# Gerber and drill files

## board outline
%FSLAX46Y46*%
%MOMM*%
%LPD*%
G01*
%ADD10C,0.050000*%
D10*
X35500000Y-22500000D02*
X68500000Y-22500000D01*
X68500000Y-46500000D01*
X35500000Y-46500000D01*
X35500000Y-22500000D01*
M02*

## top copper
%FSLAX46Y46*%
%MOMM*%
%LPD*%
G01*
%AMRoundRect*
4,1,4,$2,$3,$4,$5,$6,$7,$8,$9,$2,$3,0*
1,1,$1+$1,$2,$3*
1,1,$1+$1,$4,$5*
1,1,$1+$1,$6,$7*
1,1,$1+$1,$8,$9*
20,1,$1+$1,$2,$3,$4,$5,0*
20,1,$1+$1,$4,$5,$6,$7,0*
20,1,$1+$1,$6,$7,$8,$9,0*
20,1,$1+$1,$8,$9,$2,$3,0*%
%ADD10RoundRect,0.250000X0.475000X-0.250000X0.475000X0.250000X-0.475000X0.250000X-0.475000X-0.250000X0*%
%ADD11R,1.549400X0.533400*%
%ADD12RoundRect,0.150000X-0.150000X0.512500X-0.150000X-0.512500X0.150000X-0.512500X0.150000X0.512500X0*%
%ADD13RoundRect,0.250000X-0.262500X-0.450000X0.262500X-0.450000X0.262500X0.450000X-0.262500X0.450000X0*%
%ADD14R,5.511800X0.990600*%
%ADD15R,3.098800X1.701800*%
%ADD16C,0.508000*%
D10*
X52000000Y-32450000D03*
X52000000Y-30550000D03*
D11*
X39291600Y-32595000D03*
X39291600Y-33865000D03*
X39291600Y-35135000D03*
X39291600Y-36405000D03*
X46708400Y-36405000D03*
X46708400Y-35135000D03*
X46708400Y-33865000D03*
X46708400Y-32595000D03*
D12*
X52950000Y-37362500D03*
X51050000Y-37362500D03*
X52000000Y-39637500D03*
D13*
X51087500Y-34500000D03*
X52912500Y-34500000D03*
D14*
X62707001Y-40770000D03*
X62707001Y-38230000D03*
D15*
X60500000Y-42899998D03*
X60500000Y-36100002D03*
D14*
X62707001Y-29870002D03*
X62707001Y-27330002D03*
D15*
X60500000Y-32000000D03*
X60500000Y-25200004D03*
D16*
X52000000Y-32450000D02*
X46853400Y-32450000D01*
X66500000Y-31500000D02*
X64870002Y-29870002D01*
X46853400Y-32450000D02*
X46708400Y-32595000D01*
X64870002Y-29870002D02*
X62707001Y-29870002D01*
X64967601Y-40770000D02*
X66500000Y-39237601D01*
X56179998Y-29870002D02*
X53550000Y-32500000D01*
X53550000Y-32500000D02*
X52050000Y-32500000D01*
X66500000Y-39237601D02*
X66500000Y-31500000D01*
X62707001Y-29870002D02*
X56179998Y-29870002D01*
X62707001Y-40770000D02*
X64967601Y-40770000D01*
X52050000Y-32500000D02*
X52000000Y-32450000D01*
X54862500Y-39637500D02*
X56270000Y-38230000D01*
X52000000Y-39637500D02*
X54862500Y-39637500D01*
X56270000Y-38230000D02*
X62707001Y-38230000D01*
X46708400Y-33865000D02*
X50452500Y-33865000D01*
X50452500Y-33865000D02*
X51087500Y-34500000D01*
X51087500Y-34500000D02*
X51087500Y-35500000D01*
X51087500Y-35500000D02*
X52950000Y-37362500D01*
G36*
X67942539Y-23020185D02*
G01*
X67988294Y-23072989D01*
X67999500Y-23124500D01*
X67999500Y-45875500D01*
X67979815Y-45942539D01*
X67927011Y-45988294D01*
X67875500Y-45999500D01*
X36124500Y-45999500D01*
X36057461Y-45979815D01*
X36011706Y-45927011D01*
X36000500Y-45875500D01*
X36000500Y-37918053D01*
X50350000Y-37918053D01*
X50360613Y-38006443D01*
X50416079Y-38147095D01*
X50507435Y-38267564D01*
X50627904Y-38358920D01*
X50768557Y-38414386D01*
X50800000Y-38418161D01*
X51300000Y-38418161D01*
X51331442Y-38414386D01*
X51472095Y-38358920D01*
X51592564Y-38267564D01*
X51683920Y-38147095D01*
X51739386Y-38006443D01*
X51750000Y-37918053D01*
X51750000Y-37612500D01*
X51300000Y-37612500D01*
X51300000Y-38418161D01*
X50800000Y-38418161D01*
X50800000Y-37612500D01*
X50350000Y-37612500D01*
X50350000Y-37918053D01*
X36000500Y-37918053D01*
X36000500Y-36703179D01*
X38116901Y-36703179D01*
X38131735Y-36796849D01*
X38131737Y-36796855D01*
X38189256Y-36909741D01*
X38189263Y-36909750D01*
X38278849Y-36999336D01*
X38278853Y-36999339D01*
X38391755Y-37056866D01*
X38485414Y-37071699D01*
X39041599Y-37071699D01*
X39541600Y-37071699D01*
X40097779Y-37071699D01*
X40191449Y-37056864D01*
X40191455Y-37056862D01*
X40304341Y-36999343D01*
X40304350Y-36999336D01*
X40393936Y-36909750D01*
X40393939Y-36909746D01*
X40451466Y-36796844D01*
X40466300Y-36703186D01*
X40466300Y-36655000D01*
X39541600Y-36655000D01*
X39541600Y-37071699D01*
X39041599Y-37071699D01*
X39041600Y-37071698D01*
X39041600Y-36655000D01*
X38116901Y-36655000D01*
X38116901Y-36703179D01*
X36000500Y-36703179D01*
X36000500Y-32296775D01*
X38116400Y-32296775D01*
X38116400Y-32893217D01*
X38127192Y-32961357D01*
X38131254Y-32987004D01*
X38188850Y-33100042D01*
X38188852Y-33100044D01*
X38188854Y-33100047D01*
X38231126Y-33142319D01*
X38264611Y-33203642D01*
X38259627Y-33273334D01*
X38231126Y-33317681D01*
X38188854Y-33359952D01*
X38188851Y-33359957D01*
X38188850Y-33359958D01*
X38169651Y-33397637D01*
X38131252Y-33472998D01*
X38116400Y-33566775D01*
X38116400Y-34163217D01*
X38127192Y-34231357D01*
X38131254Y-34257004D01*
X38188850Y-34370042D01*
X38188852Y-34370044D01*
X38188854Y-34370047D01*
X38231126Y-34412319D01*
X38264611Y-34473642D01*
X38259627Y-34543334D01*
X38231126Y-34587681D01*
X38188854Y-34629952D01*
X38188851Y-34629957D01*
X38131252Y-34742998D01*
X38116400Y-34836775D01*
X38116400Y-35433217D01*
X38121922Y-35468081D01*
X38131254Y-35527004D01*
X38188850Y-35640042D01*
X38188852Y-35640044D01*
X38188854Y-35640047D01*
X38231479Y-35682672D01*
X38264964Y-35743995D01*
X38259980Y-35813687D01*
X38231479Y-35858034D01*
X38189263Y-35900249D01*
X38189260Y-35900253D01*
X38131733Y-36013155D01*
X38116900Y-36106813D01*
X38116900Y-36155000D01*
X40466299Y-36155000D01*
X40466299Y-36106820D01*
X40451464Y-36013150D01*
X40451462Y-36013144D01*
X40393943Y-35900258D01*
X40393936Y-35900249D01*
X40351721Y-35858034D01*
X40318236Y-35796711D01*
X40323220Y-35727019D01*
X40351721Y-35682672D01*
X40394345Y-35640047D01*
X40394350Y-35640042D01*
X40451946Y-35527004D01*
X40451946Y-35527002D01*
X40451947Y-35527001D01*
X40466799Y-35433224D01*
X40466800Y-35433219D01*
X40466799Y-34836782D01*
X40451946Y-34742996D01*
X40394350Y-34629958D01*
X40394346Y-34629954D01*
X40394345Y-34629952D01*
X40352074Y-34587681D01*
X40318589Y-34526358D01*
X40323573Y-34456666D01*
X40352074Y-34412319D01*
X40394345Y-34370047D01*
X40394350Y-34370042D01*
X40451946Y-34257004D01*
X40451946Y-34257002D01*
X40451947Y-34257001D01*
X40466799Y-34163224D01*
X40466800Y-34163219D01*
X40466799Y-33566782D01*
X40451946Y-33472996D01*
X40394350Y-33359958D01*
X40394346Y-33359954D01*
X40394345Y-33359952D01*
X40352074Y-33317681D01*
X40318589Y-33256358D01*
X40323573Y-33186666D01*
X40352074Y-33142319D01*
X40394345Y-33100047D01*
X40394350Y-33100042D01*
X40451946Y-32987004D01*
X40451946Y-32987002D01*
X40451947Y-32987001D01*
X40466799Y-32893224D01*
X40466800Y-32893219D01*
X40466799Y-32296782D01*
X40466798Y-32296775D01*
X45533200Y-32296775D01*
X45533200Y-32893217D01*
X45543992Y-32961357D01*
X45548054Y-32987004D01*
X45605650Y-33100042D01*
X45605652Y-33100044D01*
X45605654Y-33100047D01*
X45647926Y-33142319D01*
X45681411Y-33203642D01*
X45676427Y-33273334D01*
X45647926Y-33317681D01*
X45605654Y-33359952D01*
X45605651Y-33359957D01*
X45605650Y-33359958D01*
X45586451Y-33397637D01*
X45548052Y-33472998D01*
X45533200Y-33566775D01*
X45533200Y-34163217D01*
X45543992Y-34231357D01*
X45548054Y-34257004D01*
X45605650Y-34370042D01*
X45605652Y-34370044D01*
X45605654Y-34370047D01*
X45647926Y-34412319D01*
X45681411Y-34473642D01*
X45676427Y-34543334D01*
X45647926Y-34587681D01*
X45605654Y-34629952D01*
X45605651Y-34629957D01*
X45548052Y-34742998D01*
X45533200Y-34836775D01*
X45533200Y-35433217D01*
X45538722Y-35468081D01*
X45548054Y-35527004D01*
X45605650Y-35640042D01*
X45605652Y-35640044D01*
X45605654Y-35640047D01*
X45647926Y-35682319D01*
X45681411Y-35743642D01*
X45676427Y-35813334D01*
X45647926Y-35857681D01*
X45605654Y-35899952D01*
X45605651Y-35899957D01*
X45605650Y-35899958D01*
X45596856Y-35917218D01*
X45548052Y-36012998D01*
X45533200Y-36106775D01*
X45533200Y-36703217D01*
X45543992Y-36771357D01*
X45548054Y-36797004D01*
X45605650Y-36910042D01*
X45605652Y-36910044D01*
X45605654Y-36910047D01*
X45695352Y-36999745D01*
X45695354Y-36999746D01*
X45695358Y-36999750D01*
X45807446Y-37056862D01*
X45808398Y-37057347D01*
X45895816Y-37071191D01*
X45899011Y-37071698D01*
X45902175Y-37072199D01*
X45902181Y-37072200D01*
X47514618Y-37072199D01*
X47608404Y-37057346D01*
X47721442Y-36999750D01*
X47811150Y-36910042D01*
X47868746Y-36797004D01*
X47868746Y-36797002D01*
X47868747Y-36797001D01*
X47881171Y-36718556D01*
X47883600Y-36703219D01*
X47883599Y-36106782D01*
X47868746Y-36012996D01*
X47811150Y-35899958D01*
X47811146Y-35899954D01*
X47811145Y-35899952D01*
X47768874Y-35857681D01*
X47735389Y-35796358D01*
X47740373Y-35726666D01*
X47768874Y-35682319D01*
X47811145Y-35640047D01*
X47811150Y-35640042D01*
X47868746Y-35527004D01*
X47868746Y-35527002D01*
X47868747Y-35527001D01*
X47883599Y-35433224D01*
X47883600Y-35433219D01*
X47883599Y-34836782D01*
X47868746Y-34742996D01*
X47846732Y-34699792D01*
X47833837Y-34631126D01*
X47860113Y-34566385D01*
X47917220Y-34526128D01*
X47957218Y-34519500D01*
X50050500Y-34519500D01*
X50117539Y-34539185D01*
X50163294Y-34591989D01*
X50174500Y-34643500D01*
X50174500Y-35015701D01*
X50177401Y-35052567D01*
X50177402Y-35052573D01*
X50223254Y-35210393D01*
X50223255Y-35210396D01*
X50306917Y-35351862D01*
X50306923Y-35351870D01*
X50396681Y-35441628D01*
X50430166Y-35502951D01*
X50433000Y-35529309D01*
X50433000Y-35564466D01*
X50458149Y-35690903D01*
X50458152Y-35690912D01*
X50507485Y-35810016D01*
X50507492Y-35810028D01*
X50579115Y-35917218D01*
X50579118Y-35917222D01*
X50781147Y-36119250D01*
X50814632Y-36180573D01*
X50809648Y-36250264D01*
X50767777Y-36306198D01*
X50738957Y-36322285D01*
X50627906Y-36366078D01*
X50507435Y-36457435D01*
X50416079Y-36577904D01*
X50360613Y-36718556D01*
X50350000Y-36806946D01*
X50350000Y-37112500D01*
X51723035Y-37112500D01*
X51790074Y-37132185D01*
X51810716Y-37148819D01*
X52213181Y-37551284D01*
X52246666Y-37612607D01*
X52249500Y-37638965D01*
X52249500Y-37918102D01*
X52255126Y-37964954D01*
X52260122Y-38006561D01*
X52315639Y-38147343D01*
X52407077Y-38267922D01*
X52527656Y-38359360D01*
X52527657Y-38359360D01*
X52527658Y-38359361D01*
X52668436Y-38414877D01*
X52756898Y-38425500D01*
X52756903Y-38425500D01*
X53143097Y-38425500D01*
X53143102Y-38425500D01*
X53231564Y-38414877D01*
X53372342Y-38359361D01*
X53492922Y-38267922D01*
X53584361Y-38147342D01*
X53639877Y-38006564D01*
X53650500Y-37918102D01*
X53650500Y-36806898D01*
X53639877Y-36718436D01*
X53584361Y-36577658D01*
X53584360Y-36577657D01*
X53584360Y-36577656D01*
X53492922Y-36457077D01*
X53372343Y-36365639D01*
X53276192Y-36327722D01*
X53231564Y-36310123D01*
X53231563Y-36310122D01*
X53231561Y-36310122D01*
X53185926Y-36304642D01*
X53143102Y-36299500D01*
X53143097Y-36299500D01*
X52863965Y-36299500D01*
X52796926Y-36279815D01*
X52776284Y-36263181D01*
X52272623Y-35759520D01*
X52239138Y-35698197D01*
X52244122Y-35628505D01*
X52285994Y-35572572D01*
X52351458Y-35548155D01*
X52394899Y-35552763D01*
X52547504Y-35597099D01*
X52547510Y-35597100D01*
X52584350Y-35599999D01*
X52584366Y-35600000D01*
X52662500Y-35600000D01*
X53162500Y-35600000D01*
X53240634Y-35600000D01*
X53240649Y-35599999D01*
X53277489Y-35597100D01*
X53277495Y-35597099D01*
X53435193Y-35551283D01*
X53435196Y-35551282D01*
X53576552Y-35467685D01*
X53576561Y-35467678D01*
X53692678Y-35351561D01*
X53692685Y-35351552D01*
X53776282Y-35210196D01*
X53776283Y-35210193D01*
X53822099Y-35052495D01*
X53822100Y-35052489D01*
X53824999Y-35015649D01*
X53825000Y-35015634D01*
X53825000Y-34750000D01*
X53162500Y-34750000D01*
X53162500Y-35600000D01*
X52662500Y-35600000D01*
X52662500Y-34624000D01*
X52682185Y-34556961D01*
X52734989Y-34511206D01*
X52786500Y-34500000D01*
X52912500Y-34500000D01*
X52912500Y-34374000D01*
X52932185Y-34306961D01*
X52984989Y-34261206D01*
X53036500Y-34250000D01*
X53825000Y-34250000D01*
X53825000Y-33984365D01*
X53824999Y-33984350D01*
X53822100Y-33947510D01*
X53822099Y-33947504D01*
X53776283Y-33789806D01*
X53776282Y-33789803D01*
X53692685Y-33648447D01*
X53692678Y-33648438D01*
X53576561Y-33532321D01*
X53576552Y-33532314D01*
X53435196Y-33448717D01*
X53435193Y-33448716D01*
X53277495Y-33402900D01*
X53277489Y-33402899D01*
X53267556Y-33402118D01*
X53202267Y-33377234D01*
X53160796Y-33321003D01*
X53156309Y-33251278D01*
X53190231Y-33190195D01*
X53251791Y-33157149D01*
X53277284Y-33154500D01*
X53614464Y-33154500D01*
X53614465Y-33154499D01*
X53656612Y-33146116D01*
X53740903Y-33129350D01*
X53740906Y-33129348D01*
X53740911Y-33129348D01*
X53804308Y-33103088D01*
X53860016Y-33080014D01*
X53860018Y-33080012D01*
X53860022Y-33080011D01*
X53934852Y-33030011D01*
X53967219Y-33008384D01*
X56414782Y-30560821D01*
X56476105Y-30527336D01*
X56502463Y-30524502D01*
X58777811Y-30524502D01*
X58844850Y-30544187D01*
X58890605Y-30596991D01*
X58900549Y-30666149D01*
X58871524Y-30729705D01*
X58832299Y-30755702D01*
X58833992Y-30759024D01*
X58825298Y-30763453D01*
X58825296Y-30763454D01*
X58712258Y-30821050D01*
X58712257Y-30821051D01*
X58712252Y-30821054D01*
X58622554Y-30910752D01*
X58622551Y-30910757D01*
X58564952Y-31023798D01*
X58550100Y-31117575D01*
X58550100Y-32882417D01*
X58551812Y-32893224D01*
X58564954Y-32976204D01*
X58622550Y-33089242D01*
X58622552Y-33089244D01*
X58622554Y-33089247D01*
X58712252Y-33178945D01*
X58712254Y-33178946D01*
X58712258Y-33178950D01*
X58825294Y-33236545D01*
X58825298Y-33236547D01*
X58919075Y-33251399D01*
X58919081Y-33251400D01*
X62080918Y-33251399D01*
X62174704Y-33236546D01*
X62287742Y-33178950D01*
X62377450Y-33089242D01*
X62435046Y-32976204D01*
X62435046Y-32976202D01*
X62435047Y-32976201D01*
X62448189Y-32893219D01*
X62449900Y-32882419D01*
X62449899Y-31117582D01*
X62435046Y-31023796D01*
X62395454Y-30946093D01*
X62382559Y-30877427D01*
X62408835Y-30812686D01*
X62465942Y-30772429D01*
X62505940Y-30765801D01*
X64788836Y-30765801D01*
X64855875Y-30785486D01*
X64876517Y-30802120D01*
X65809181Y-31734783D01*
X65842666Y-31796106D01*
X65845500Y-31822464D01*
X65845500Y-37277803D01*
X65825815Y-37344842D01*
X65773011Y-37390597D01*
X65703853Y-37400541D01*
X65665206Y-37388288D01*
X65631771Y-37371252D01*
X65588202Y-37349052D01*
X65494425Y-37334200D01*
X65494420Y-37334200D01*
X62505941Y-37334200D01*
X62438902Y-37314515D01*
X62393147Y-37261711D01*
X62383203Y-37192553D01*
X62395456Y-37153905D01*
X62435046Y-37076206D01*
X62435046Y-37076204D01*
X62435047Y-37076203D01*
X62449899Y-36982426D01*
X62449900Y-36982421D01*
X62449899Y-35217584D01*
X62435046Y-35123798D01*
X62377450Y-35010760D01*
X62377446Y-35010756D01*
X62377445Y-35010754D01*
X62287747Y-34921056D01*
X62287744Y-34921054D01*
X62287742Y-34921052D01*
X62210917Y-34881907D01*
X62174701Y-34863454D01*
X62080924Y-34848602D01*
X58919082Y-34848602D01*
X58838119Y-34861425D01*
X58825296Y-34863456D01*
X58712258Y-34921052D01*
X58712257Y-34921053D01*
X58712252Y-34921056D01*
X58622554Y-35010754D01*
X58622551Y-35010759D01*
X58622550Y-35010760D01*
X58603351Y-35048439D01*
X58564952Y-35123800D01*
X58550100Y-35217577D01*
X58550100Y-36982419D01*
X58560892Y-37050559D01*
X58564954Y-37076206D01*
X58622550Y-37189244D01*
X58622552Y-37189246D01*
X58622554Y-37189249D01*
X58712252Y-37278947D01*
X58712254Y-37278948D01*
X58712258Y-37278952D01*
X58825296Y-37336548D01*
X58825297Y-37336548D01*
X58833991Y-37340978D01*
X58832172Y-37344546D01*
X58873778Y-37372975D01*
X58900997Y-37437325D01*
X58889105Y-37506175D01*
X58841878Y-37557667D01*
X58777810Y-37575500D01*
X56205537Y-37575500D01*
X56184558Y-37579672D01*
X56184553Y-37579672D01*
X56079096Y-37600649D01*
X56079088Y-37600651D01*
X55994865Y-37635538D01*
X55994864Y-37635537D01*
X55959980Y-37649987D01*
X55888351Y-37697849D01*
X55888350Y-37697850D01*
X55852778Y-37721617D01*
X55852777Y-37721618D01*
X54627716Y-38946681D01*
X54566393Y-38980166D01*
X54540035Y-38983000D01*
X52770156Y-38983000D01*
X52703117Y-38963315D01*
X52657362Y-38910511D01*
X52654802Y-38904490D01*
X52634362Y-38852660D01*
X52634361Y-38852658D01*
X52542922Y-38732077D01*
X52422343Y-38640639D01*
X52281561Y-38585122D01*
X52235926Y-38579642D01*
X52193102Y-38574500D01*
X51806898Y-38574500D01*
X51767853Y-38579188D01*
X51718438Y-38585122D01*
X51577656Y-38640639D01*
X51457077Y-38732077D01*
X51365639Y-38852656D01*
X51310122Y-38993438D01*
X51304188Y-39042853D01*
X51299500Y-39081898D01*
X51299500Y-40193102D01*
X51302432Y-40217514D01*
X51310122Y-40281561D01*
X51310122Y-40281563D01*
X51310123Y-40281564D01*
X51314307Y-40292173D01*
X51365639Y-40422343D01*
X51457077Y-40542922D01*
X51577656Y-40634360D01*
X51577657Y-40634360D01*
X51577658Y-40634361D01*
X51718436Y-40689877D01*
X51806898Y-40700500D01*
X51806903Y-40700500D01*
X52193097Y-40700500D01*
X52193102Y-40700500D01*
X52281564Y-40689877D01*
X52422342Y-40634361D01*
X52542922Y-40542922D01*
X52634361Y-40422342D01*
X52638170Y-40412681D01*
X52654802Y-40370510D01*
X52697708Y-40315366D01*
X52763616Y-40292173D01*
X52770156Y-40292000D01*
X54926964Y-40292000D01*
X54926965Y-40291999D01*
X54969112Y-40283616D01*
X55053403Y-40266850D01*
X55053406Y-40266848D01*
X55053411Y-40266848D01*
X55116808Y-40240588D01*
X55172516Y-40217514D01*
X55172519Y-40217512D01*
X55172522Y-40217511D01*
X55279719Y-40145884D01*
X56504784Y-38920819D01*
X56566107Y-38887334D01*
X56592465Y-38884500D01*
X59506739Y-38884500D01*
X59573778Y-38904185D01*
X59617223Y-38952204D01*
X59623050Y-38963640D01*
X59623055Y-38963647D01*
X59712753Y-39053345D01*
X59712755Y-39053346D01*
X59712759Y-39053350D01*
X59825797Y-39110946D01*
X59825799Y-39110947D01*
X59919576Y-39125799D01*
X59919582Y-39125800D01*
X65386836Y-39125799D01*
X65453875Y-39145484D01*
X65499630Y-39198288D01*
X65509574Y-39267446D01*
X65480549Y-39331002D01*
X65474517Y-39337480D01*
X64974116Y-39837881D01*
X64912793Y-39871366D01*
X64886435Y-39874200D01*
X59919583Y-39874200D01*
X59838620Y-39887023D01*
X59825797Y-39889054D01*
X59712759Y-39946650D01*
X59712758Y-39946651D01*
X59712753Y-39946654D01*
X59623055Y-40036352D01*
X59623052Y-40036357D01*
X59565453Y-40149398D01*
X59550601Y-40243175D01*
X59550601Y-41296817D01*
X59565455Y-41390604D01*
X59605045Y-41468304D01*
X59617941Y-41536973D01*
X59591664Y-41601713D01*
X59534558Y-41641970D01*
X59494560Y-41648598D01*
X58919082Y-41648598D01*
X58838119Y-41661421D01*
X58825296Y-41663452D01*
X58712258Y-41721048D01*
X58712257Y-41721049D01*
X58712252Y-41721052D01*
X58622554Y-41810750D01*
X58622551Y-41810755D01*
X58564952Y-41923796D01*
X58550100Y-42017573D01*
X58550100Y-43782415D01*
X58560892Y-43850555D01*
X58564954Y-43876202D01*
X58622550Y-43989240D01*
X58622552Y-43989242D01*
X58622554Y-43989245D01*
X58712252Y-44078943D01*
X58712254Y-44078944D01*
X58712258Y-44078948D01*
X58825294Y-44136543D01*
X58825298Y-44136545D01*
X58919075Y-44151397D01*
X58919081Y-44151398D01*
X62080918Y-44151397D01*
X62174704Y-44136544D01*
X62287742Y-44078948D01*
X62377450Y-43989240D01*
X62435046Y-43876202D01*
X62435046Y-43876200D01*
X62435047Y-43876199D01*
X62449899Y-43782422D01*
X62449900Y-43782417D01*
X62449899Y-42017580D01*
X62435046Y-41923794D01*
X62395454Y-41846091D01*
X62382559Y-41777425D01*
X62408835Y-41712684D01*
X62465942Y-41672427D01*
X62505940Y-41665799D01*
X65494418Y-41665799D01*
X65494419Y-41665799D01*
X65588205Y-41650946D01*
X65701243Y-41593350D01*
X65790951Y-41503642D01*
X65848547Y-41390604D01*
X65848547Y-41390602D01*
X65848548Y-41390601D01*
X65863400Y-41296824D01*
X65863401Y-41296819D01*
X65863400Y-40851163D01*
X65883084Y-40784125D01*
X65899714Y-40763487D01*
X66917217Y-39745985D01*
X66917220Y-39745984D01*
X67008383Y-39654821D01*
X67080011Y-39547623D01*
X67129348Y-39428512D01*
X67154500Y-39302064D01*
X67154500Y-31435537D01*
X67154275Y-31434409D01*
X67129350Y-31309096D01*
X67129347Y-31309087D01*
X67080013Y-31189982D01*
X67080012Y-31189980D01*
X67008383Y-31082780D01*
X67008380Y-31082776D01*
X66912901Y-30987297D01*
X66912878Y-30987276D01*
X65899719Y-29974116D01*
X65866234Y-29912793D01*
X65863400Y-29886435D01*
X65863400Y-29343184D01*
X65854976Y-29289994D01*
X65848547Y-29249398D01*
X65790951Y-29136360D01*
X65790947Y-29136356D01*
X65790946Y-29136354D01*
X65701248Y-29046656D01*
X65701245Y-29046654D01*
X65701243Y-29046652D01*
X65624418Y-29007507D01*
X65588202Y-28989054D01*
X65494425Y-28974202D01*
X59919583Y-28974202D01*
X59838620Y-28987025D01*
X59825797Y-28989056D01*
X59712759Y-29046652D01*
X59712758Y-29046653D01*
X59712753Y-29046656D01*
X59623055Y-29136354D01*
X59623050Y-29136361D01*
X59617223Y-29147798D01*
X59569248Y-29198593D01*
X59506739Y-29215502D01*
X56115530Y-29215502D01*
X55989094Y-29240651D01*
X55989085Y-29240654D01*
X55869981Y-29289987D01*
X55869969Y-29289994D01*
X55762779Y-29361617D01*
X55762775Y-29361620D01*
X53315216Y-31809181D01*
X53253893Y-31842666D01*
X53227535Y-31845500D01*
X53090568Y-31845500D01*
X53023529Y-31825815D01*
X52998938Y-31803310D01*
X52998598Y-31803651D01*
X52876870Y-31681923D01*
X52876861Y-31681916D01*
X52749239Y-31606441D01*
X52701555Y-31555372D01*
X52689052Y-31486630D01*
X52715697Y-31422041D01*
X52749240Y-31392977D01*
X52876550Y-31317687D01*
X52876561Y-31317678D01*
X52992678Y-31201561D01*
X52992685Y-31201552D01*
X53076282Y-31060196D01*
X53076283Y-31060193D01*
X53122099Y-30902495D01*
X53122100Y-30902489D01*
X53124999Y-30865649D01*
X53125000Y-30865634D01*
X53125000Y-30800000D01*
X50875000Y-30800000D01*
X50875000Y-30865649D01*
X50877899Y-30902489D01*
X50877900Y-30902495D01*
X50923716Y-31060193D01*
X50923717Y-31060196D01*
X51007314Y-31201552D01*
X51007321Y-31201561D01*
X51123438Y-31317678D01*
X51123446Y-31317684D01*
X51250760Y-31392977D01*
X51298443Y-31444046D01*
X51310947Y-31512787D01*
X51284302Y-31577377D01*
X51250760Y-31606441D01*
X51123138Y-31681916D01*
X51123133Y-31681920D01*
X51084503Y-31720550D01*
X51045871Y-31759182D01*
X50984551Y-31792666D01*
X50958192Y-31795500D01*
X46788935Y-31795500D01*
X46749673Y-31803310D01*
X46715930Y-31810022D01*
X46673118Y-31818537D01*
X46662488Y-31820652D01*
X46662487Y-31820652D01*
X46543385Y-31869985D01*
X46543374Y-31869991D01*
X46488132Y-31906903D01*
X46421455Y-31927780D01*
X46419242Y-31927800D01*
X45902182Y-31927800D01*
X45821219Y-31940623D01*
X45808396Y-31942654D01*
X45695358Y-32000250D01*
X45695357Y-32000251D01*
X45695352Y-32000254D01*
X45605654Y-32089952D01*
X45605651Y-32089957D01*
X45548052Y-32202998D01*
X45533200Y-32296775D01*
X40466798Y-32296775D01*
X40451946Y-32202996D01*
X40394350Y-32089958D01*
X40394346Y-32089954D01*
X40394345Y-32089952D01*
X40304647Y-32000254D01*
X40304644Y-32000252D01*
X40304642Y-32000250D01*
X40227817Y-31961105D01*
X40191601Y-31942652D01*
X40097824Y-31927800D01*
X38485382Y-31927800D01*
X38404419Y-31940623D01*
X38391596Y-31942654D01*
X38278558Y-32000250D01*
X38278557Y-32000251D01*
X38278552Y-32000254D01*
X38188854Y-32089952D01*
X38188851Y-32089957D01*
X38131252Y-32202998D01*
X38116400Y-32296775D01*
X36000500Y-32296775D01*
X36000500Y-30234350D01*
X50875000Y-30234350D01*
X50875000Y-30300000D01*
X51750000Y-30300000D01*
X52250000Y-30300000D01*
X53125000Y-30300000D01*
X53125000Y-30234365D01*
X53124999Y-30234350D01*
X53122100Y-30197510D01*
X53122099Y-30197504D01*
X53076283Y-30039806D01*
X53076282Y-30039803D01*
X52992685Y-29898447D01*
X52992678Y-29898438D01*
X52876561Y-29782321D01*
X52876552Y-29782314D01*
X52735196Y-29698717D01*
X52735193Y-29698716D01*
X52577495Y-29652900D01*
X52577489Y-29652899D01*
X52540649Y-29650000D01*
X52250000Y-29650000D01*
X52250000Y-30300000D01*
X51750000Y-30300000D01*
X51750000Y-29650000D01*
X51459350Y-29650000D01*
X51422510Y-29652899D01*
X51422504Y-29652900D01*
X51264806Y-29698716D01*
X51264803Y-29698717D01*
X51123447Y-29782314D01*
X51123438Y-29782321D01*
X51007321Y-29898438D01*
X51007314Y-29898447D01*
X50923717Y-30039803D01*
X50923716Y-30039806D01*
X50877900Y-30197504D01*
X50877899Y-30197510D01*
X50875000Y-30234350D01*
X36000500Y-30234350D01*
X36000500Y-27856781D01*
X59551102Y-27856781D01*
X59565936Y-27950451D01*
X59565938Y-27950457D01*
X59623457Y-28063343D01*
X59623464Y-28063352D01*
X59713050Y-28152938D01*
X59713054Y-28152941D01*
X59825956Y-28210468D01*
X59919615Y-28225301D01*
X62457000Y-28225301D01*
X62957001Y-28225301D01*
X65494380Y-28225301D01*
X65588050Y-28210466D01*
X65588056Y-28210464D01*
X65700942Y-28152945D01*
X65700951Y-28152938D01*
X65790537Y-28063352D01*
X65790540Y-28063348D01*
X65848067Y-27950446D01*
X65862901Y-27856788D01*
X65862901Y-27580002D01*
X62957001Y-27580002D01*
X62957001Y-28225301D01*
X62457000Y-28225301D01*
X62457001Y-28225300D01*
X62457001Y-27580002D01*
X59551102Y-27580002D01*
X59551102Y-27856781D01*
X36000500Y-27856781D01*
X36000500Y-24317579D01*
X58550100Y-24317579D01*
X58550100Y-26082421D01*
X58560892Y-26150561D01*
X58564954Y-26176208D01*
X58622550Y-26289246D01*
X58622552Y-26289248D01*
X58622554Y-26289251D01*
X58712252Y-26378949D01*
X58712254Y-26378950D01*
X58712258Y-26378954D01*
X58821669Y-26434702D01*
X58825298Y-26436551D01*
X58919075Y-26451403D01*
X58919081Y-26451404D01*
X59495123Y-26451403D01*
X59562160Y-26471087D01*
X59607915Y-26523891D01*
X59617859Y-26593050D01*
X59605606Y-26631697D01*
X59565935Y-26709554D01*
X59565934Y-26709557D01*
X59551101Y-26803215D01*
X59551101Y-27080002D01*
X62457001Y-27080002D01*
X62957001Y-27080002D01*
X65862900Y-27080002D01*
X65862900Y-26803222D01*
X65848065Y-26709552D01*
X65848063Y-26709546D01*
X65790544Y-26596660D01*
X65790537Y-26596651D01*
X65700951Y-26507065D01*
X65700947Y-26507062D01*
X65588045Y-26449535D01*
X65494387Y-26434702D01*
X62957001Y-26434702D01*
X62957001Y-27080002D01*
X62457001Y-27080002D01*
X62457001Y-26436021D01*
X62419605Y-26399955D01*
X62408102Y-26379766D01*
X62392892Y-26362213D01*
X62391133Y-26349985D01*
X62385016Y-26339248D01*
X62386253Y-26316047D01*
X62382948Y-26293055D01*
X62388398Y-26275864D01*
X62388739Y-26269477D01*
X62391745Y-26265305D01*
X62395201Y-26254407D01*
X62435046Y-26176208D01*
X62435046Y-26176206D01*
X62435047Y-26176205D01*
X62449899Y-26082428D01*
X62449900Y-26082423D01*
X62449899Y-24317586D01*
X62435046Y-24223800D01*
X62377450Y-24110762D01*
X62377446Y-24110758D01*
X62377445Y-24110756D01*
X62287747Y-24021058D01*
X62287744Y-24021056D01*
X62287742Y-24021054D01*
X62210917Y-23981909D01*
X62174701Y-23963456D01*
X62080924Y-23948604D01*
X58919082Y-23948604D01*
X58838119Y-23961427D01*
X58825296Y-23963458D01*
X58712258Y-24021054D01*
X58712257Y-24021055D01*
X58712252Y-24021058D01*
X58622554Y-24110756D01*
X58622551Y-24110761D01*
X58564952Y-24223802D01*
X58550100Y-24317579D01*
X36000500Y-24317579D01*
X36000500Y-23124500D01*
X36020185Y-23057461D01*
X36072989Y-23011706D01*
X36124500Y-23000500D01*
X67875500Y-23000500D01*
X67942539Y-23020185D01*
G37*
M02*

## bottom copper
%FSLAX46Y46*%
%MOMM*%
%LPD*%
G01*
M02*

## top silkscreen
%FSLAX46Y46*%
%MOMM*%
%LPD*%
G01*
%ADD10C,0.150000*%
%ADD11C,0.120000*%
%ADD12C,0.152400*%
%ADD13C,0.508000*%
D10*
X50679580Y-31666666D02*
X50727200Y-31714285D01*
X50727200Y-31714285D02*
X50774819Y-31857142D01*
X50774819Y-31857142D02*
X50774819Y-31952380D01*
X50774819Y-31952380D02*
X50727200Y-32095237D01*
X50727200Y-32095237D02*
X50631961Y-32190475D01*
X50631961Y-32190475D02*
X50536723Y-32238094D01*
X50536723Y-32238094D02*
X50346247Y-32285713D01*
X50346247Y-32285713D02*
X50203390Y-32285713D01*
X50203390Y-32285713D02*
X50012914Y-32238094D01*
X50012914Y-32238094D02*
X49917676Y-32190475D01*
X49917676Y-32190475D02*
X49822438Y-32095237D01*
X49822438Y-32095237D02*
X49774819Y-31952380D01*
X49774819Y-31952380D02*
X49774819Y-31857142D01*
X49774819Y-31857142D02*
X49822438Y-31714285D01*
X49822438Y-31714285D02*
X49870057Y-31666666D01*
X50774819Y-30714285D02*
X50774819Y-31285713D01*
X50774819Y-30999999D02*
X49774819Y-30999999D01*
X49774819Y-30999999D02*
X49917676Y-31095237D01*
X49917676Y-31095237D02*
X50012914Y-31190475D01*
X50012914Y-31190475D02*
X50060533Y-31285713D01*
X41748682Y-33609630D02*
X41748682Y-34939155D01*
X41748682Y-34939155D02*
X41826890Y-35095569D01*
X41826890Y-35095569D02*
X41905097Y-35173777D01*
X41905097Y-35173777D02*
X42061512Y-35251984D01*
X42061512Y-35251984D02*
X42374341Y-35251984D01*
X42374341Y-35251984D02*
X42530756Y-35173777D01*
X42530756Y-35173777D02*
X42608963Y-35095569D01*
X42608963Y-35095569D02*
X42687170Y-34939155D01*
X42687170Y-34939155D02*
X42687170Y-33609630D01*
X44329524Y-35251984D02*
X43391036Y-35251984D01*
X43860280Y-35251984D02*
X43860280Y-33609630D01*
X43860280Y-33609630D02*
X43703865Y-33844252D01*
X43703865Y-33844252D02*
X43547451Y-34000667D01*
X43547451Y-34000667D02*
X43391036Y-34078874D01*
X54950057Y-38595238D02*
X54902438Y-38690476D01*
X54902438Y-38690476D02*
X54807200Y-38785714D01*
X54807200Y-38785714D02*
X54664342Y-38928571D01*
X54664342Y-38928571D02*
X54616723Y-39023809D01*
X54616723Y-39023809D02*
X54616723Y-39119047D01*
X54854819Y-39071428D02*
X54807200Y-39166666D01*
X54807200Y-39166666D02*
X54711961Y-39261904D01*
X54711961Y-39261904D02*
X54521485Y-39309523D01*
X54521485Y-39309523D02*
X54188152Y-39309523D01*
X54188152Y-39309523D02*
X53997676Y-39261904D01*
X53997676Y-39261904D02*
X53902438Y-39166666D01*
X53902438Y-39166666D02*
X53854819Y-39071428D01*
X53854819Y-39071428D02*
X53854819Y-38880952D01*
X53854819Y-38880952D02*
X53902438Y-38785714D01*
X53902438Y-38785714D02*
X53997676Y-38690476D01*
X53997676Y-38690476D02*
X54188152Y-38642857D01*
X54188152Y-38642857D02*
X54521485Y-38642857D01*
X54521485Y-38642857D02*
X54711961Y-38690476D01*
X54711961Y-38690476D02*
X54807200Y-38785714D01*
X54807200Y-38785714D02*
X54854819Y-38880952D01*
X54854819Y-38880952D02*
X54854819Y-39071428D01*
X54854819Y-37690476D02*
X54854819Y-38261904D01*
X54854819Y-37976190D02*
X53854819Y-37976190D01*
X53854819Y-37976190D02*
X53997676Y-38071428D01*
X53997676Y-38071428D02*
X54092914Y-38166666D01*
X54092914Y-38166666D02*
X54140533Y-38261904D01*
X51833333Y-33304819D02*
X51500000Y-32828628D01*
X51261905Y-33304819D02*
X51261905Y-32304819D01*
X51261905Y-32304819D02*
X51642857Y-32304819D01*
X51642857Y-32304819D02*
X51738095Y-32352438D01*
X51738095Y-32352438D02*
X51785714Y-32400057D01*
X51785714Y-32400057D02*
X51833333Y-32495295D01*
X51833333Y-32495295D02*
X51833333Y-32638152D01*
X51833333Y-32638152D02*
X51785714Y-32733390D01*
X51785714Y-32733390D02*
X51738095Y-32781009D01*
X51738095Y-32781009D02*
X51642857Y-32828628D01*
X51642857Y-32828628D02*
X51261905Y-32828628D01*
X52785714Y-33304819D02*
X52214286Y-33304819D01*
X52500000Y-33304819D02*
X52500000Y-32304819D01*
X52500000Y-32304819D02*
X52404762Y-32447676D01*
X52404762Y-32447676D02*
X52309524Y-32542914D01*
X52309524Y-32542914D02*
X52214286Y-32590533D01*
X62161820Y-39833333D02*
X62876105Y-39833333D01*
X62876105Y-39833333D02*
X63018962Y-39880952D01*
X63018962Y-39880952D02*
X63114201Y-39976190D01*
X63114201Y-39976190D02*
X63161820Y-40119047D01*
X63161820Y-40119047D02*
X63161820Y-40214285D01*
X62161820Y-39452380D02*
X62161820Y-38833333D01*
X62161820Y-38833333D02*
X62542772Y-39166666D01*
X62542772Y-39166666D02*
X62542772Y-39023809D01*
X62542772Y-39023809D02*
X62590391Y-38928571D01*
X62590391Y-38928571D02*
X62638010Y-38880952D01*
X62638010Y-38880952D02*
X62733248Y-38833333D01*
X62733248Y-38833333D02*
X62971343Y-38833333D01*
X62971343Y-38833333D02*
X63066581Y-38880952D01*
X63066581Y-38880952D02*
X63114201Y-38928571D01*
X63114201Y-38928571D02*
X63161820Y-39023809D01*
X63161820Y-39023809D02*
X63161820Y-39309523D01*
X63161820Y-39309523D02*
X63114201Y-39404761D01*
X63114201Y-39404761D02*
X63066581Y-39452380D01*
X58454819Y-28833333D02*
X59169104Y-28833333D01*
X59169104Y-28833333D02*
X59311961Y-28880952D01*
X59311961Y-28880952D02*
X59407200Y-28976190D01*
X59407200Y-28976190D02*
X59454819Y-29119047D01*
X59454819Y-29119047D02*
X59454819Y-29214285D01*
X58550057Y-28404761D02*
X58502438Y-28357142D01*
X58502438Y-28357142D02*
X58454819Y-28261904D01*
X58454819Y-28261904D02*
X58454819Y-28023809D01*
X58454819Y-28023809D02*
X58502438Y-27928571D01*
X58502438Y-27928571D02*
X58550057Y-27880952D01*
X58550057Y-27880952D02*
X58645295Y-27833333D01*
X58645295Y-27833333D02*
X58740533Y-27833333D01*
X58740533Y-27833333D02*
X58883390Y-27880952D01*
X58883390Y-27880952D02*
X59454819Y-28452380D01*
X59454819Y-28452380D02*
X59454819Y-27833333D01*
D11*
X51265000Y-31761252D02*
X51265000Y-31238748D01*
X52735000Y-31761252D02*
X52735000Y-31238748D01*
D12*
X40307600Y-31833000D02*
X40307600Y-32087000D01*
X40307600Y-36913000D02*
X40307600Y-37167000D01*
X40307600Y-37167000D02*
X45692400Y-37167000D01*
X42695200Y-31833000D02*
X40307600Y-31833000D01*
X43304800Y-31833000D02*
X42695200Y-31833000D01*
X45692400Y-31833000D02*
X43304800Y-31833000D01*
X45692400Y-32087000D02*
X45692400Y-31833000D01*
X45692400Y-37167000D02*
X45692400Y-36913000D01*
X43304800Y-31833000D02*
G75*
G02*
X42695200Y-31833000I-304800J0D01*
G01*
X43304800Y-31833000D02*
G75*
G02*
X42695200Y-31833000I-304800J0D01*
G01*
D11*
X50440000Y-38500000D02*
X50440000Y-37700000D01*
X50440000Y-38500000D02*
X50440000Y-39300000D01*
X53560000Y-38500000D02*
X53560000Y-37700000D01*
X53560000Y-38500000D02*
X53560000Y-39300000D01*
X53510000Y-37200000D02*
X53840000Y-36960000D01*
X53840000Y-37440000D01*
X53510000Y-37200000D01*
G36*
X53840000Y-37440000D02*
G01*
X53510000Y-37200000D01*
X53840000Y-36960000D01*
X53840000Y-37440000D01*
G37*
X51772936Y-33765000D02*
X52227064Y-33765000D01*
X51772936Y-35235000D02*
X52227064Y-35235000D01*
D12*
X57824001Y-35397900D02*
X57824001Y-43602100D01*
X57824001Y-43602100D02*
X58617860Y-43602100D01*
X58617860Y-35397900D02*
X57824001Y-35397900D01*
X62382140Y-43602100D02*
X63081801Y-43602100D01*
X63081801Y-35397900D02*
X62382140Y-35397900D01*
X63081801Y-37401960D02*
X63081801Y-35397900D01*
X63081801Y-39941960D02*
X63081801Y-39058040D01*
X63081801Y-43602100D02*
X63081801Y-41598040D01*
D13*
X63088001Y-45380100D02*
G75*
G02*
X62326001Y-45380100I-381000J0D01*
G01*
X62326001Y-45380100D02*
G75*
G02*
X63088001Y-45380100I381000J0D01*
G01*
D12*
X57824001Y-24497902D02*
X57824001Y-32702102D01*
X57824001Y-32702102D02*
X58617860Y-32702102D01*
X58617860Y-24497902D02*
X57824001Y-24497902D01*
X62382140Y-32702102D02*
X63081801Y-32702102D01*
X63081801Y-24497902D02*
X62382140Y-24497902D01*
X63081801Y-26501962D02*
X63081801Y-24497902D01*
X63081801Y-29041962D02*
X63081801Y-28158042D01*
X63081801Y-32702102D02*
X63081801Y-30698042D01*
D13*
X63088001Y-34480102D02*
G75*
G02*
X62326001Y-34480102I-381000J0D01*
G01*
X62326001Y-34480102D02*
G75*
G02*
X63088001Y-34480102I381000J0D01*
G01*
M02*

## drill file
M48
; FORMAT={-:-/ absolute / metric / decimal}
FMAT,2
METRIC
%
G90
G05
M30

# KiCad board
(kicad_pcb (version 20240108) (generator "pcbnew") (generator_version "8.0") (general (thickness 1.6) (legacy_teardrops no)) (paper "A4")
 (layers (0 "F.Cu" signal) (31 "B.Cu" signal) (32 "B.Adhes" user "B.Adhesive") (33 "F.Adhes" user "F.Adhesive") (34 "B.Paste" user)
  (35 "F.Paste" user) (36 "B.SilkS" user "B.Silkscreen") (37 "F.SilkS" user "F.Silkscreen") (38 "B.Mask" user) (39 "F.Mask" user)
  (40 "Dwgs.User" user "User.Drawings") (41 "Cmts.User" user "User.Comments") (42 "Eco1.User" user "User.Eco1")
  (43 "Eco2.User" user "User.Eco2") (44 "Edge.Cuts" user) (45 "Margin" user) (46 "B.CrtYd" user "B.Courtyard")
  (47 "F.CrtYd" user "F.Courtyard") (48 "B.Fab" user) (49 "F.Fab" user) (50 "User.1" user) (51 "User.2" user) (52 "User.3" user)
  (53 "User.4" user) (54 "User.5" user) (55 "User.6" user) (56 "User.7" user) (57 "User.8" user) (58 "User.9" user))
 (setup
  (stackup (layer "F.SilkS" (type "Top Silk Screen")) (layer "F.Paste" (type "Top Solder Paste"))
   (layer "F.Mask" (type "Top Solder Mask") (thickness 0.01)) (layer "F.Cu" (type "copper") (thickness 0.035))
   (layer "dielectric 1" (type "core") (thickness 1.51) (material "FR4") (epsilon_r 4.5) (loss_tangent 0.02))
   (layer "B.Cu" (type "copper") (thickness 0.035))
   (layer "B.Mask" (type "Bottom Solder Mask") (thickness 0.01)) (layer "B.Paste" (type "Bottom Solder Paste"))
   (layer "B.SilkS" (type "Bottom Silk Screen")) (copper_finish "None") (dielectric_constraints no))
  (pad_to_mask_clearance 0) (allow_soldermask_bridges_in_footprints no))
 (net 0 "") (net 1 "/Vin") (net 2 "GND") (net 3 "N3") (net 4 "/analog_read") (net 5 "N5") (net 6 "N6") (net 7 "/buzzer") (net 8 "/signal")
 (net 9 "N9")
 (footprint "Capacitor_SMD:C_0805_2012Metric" (layer "F.Cu") (at 52 31.5 90)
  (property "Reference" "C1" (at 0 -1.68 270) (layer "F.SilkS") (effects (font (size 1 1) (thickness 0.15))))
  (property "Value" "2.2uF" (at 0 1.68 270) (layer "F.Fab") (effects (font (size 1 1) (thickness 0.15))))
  (fp_line (start -0.261252 -0.735) (end 0.261252 -0.735) (stroke (width 0.12) (type solid)) (layer "F.SilkS"))
  (fp_line (start -0.261252 0.735) (end 0.261252 0.735) (stroke (width 0.12) (type solid)) (layer "F.SilkS"))
  (pad "1" smd roundrect (at -0.95 0 90) (size 1 1.45) (layers "F.Cu" "F.Paste" "F.Mask") (roundrect_rratio 0.25) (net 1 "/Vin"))
  (pad "2" smd roundrect (at 0.95 0 90) (size 1 1.45) (layers "F.Cu" "F.Paste" "F.Mask") (roundrect_rratio 0.25) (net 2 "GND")))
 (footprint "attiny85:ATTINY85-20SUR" (layer "F.Cu") (at 43 34.5)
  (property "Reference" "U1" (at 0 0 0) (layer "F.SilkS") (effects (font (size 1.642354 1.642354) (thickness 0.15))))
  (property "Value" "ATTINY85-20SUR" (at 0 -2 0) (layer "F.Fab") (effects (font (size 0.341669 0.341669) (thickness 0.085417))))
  (fp_line (start -2.6924 -2.667) (end -2.6924 -2.413) (stroke (width 0.1524) (type solid)) (layer "F.SilkS"))
  (fp_line (start -2.6924 2.413) (end -2.6924 2.667) (stroke (width 0.1524) (type solid)) (layer "F.SilkS"))
  (fp_line (start -2.6924 2.667) (end 2.6924 2.667) (stroke (width 0.1524) (type solid)) (layer "F.SilkS"))
  (fp_line (start -0.3048 -2.667) (end -2.6924 -2.667) (stroke (width 0.1524) (type solid)) (layer "F.SilkS"))
  (fp_line (start 0.3048 -2.667) (end -0.3048 -2.667) (stroke (width 0.1524) (type solid)) (layer "F.SilkS"))
  (fp_line (start 2.6924 -2.667) (end 0.3048 -2.667) (stroke (width 0.1524) (type solid)) (layer "F.SilkS"))
  (fp_line (start 2.6924 -2.413) (end 2.6924 -2.667) (stroke (width 0.1524) (type solid)) (layer "F.SilkS"))
  (fp_line (start 2.6924 2.667) (end 2.6924 2.413) (stroke (width 0.1524) (type solid)) (layer "F.SilkS"))
  (fp_arc (start 0.3048 -2.667) (mid 0 -2.3622) (end -0.3048 -2.667) (stroke (width 0.1524) (type solid)) (layer "F.SilkS"))
  (fp_arc (start 0.3048 -2.667) (mid 0 -2.3622) (end -0.3048 -2.667) (stroke (width 0.1524) (type solid)) (layer "F.SilkS"))
  (pad "1" smd rect (at -3.7084 -1.905) (size 1.5494 0.5334) (layers "F.Cu" "F.Paste" "F.Mask") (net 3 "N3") (solder_mask_margin 0.102))
  (pad "2" smd rect (at -3.7084 -0.635) (size 1.5494 0.5334) (layers "F.Cu" "F.Paste" "F.Mask") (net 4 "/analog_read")
   (solder_mask_margin 0.102))
  (pad "3" smd rect (at -3.7084 0.635) (size 1.5494 0.5334) (layers "F.Cu" "F.Paste" "F.Mask") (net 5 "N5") (solder_mask_margin 0.102))
  (pad "4" smd rect (at -3.7084 1.905) (size 1.5494 0.5334) (layers "F.Cu" "F.Paste" "F.Mask") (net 2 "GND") (solder_mask_margin 0.102))
  (pad "5" smd rect (at 3.7084 1.905) (size 1.5494 0.5334) (layers "F.Cu" "F.Paste" "F.Mask") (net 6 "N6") (solder_mask_margin 0.102))
  (pad "6" smd rect (at 3.7084 0.635) (size 1.5494 0.5334) (layers "F.Cu" "F.Paste" "F.Mask") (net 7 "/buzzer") (solder_mask_margin 0.102))
  (pad "7" smd rect (at 3.7084 -0.635) (size 1.5494 0.5334) (layers "F.Cu" "F.Paste" "F.Mask") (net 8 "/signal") (solder_mask_margin 0.102))
  (pad "8" smd rect (at 3.7084 -1.905) (size 1.5494 0.5334) (layers "F.Cu" "F.Paste" "F.Mask") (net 1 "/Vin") (solder_mask_margin 0.102)))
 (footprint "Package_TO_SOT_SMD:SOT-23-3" (layer "F.Cu") (at 52 38.5 -90)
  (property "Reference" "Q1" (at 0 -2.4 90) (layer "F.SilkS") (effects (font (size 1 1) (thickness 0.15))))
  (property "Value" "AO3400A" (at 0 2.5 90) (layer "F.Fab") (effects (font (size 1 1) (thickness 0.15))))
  (fp_line (start 0 1.56) (end -0.8 1.56) (stroke (width 0.12) (type solid)) (layer "F.SilkS"))
  (fp_line (start 0 1.56) (end 0.8 1.56) (stroke (width 0.12) (type solid)) (layer "F.SilkS"))
  (fp_line (start 0 -1.56) (end -0.8 -1.56) (stroke (width 0.12) (type solid)) (layer "F.SilkS"))
  (fp_line (start 0 -1.56) (end 0.8 -1.56) (stroke (width 0.12) (type solid)) (layer "F.SilkS"))
  (fp_poly
   (pts (xy -1.3 -1.51) (xy -1.54 -1.84) (xy -1.06 -1.84) (xy -1.3 -1.51)) (stroke (width 0.12) (type solid)) (fill solid) (layer "F.SilkS"))
  (pad "1" smd roundrect (at -1.1375 -0.95 270) (size 1.325 0.6) (layers "F.Cu" "F.Paste" "F.Mask") (roundrect_rratio 0.25)
   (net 8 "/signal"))
  (pad "2" smd roundrect (at -1.1375 0.95 270) (size 1.325 0.6) (layers "F.Cu" "F.Paste" "F.Mask") (roundrect_rratio 0.25) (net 2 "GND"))
  (pad "3" smd roundrect (at 1.1375 0 270) (size 1.325 0.6) (layers "F.Cu" "F.Paste" "F.Mask") (roundrect_rratio 0.25) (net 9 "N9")))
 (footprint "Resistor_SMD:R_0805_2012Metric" (layer "F.Cu") (at 52 34.5)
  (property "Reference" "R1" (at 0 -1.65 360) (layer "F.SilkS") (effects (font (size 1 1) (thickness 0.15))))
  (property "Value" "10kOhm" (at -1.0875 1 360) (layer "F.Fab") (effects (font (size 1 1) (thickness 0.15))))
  (fp_line (start -0.227064 -0.735) (end 0.227064 -0.735) (stroke (width 0.12) (type solid)) (layer "F.SilkS"))
  (fp_line (start -0.227064 0.735) (end 0.227064 0.735) (stroke (width 0.12) (type solid)) (layer "F.SilkS"))
  (pad "1" smd roundrect (at -0.9125 0) (size 1.025 1.4) (layers "F.Cu" "F.Paste" "F.Mask") (roundrect_rratio 0.243902) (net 8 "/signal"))
  (pad "2" smd roundrect (at 0.9125 0) (size 1.025 1.4) (layers "F.Cu" "F.Paste" "F.Mask") (roundrect_rratio 0.243902) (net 2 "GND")))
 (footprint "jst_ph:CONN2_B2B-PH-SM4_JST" (layer "F.Cu") (at 60.452901 39.5 90)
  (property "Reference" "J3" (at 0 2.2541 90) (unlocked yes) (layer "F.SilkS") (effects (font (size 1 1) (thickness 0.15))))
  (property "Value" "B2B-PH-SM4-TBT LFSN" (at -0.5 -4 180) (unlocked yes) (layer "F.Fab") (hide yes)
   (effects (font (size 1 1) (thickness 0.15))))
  (fp_line (start 4.1021 -2.6289) (end -4.1021 -2.6289) (stroke (width 0.1524) (type solid)) (layer "F.SilkS"))
  (fp_line (start -4.1021 -2.6289) (end -4.1021 -1.835041) (stroke (width 0.1524) (type solid)) (layer "F.SilkS"))
  (fp_line (start 4.1021 -1.835041) (end 4.1021 -2.6289) (stroke (width 0.1524) (type solid)) (layer "F.SilkS"))
  (fp_line (start -4.1021 1.929239) (end -4.1021 2.6289) (stroke (width 0.1524) (type solid)) (layer "F.SilkS"))
  (fp_line (start 4.1021 2.6289) (end 4.1021 1.929239) (stroke (width 0.1524) (type solid)) (layer "F.SilkS"))
  (fp_line (start 2.09804 2.6289) (end 4.1021 2.6289) (stroke (width 0.1524) (type solid)) (layer "F.SilkS"))
  (fp_line (start -0.44196 2.6289) (end 0.44196 2.6289) (stroke (width 0.1524) (type solid)) (layer "F.SilkS"))
  (fp_line (start -4.1021 2.6289) (end -2.09804 2.6289) (stroke (width 0.1524) (type solid)) (layer "F.SilkS"))
  (fp_circle (center -5.8801 2.2541) (end -5.4991 2.2541) (stroke (width 0.508) (type solid)) (fill none) (layer "F.SilkS"))
  (pad "1" smd rect (at -1.27 2.2541 90) (size 0.9906 5.5118) (layers "F.Cu" "F.Paste" "F.Mask") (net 1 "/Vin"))
  (pad "2" smd rect (at 1.27 2.2541 90) (size 0.9906 5.5118) (layers "F.Cu" "F.Paste" "F.Mask") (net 9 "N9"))
  (pad "3" smd rect (at -3.399998 0.047099 90) (size 1.7018 3.0988) (layers "F.Cu" "F.Paste" "F.Mask"))
  (pad "4" smd rect (at 3.399998 0.047099 90) (size 1.7018 3.0988) (layers "F.Cu" "F.Paste" "F.Mask")))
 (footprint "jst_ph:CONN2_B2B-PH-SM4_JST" (layer "F.Cu") (at 60.452901 28.600002 90)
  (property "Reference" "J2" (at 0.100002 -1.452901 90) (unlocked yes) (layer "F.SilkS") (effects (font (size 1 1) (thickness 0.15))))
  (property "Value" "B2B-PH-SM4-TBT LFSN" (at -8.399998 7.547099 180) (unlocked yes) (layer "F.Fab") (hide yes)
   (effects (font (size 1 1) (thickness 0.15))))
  (fp_line (start 4.1021 -2.6289) (end -4.1021 -2.6289) (stroke (width 0.1524) (type solid)) (layer "F.SilkS"))
  (fp_line (start -4.1021 -2.6289) (end -4.1021 -1.835041) (stroke (width 0.1524) (type solid)) (layer "F.SilkS"))
  (fp_line (start 4.1021 -1.835041) (end 4.1021 -2.6289) (stroke (width 0.1524) (type solid)) (layer "F.SilkS"))
  (fp_line (start -4.1021 1.929239) (end -4.1021 2.6289) (stroke (width 0.1524) (type solid)) (layer "F.SilkS"))
  (fp_line (start 4.1021 2.6289) (end 4.1021 1.929239) (stroke (width 0.1524) (type solid)) (layer "F.SilkS"))
  (fp_line (start 2.09804 2.6289) (end 4.1021 2.6289) (stroke (width 0.1524) (type solid)) (layer "F.SilkS"))
  (fp_line (start -0.44196 2.6289) (end 0.44196 2.6289) (stroke (width 0.1524) (type solid)) (layer "F.SilkS"))
  (fp_line (start -4.1021 2.6289) (end -2.09804 2.6289) (stroke (width 0.1524) (type solid)) (layer "F.SilkS"))
  (fp_circle (center -5.8801 2.2541) (end -5.4991 2.2541) (stroke (width 0.508) (type solid)) (fill none) (layer "F.SilkS"))
  (pad "1" smd rect (at -1.27 2.2541 90) (size 0.9906 5.5118) (layers "F.Cu" "F.Paste" "F.Mask") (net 1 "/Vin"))
  (pad "2" smd rect (at 1.27 2.2541 90) (size 0.9906 5.5118) (layers "F.Cu" "F.Paste" "F.Mask") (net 2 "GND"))
  (pad "3" smd rect (at -3.399998 0.047099 90) (size 1.7018 3.0988) (layers "F.Cu" "F.Paste" "F.Mask"))
  (pad "4" smd rect (at 3.399998 0.047099 90) (size 1.7018 3.0988) (layers "F.Cu" "F.Paste" "F.Mask")))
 (gr_rect (start 35.5 22.5) (end 68.5 46.5) (stroke (width 0.05) (type default)) (fill none) (layer "Edge.Cuts"))
 (segment (start 52 32.45) (end 46.8534 32.45) (width 0.508) (layer "F.Cu") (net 1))
 (segment (start 66.5 31.5) (end 64.870002 29.870002) (width 0.508) (layer "F.Cu") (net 1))
 (segment (start 46.8534 32.45) (end 46.7084 32.595) (width 0.508) (layer "F.Cu") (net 1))
 (segment (start 64.870002 29.870002) (end 62.707001 29.870002) (width 0.508) (layer "F.Cu") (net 1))
 (segment (start 64.967601 40.77) (end 66.5 39.237601) (width 0.508) (layer "F.Cu") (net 1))
 (segment (start 56.179998 29.870002) (end 53.55 32.5) (width 0.508) (layer "F.Cu") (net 1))
 (segment (start 53.55 32.5) (end 52.05 32.5) (width 0.508) (layer "F.Cu") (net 1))
 (segment (start 66.5 39.237601) (end 66.5 31.5) (width 0.508) (layer "F.Cu") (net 1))
 (segment (start 62.707001 29.870002) (end 56.179998 29.870002) (width 0.508) (layer "F.Cu") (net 1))
 (segment (start 62.707001 40.77) (end 64.967601 40.77) (width 0.508) (layer "F.Cu") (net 1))
 (segment (start 52.05 32.5) (end 52 32.45) (width 0.508) (layer "F.Cu") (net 1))
 (segment (start 54.8625 39.6375) (end 56.27 38.23) (width 0.508) (layer "F.Cu") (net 9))
 (segment (start 52 39.6375) (end 54.8625 39.6375) (width 0.508) (layer "F.Cu") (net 9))
 (segment (start 56.27 38.23) (end 62.707001 38.23) (width 0.508) (layer "F.Cu") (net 9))
 (segment (start 46.7084 33.865) (end 50.4525 33.865) (width 0.508) (layer "F.Cu") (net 8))
 (segment (start 50.4525 33.865) (end 51.0875 34.5) (width 0.508) (layer "F.Cu") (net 8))
 (segment (start 51.0875 34.5) (end 51.0875 35.5) (width 0.508) (layer "F.Cu") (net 8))
 (segment (start 51.0875 35.5) (end 52.95 37.3625) (width 0.508) (layer "F.Cu") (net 8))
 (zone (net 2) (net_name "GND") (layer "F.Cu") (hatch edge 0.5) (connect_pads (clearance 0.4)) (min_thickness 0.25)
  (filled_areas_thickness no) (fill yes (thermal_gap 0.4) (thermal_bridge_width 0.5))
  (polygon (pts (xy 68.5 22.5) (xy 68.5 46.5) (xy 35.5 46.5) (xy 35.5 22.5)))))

